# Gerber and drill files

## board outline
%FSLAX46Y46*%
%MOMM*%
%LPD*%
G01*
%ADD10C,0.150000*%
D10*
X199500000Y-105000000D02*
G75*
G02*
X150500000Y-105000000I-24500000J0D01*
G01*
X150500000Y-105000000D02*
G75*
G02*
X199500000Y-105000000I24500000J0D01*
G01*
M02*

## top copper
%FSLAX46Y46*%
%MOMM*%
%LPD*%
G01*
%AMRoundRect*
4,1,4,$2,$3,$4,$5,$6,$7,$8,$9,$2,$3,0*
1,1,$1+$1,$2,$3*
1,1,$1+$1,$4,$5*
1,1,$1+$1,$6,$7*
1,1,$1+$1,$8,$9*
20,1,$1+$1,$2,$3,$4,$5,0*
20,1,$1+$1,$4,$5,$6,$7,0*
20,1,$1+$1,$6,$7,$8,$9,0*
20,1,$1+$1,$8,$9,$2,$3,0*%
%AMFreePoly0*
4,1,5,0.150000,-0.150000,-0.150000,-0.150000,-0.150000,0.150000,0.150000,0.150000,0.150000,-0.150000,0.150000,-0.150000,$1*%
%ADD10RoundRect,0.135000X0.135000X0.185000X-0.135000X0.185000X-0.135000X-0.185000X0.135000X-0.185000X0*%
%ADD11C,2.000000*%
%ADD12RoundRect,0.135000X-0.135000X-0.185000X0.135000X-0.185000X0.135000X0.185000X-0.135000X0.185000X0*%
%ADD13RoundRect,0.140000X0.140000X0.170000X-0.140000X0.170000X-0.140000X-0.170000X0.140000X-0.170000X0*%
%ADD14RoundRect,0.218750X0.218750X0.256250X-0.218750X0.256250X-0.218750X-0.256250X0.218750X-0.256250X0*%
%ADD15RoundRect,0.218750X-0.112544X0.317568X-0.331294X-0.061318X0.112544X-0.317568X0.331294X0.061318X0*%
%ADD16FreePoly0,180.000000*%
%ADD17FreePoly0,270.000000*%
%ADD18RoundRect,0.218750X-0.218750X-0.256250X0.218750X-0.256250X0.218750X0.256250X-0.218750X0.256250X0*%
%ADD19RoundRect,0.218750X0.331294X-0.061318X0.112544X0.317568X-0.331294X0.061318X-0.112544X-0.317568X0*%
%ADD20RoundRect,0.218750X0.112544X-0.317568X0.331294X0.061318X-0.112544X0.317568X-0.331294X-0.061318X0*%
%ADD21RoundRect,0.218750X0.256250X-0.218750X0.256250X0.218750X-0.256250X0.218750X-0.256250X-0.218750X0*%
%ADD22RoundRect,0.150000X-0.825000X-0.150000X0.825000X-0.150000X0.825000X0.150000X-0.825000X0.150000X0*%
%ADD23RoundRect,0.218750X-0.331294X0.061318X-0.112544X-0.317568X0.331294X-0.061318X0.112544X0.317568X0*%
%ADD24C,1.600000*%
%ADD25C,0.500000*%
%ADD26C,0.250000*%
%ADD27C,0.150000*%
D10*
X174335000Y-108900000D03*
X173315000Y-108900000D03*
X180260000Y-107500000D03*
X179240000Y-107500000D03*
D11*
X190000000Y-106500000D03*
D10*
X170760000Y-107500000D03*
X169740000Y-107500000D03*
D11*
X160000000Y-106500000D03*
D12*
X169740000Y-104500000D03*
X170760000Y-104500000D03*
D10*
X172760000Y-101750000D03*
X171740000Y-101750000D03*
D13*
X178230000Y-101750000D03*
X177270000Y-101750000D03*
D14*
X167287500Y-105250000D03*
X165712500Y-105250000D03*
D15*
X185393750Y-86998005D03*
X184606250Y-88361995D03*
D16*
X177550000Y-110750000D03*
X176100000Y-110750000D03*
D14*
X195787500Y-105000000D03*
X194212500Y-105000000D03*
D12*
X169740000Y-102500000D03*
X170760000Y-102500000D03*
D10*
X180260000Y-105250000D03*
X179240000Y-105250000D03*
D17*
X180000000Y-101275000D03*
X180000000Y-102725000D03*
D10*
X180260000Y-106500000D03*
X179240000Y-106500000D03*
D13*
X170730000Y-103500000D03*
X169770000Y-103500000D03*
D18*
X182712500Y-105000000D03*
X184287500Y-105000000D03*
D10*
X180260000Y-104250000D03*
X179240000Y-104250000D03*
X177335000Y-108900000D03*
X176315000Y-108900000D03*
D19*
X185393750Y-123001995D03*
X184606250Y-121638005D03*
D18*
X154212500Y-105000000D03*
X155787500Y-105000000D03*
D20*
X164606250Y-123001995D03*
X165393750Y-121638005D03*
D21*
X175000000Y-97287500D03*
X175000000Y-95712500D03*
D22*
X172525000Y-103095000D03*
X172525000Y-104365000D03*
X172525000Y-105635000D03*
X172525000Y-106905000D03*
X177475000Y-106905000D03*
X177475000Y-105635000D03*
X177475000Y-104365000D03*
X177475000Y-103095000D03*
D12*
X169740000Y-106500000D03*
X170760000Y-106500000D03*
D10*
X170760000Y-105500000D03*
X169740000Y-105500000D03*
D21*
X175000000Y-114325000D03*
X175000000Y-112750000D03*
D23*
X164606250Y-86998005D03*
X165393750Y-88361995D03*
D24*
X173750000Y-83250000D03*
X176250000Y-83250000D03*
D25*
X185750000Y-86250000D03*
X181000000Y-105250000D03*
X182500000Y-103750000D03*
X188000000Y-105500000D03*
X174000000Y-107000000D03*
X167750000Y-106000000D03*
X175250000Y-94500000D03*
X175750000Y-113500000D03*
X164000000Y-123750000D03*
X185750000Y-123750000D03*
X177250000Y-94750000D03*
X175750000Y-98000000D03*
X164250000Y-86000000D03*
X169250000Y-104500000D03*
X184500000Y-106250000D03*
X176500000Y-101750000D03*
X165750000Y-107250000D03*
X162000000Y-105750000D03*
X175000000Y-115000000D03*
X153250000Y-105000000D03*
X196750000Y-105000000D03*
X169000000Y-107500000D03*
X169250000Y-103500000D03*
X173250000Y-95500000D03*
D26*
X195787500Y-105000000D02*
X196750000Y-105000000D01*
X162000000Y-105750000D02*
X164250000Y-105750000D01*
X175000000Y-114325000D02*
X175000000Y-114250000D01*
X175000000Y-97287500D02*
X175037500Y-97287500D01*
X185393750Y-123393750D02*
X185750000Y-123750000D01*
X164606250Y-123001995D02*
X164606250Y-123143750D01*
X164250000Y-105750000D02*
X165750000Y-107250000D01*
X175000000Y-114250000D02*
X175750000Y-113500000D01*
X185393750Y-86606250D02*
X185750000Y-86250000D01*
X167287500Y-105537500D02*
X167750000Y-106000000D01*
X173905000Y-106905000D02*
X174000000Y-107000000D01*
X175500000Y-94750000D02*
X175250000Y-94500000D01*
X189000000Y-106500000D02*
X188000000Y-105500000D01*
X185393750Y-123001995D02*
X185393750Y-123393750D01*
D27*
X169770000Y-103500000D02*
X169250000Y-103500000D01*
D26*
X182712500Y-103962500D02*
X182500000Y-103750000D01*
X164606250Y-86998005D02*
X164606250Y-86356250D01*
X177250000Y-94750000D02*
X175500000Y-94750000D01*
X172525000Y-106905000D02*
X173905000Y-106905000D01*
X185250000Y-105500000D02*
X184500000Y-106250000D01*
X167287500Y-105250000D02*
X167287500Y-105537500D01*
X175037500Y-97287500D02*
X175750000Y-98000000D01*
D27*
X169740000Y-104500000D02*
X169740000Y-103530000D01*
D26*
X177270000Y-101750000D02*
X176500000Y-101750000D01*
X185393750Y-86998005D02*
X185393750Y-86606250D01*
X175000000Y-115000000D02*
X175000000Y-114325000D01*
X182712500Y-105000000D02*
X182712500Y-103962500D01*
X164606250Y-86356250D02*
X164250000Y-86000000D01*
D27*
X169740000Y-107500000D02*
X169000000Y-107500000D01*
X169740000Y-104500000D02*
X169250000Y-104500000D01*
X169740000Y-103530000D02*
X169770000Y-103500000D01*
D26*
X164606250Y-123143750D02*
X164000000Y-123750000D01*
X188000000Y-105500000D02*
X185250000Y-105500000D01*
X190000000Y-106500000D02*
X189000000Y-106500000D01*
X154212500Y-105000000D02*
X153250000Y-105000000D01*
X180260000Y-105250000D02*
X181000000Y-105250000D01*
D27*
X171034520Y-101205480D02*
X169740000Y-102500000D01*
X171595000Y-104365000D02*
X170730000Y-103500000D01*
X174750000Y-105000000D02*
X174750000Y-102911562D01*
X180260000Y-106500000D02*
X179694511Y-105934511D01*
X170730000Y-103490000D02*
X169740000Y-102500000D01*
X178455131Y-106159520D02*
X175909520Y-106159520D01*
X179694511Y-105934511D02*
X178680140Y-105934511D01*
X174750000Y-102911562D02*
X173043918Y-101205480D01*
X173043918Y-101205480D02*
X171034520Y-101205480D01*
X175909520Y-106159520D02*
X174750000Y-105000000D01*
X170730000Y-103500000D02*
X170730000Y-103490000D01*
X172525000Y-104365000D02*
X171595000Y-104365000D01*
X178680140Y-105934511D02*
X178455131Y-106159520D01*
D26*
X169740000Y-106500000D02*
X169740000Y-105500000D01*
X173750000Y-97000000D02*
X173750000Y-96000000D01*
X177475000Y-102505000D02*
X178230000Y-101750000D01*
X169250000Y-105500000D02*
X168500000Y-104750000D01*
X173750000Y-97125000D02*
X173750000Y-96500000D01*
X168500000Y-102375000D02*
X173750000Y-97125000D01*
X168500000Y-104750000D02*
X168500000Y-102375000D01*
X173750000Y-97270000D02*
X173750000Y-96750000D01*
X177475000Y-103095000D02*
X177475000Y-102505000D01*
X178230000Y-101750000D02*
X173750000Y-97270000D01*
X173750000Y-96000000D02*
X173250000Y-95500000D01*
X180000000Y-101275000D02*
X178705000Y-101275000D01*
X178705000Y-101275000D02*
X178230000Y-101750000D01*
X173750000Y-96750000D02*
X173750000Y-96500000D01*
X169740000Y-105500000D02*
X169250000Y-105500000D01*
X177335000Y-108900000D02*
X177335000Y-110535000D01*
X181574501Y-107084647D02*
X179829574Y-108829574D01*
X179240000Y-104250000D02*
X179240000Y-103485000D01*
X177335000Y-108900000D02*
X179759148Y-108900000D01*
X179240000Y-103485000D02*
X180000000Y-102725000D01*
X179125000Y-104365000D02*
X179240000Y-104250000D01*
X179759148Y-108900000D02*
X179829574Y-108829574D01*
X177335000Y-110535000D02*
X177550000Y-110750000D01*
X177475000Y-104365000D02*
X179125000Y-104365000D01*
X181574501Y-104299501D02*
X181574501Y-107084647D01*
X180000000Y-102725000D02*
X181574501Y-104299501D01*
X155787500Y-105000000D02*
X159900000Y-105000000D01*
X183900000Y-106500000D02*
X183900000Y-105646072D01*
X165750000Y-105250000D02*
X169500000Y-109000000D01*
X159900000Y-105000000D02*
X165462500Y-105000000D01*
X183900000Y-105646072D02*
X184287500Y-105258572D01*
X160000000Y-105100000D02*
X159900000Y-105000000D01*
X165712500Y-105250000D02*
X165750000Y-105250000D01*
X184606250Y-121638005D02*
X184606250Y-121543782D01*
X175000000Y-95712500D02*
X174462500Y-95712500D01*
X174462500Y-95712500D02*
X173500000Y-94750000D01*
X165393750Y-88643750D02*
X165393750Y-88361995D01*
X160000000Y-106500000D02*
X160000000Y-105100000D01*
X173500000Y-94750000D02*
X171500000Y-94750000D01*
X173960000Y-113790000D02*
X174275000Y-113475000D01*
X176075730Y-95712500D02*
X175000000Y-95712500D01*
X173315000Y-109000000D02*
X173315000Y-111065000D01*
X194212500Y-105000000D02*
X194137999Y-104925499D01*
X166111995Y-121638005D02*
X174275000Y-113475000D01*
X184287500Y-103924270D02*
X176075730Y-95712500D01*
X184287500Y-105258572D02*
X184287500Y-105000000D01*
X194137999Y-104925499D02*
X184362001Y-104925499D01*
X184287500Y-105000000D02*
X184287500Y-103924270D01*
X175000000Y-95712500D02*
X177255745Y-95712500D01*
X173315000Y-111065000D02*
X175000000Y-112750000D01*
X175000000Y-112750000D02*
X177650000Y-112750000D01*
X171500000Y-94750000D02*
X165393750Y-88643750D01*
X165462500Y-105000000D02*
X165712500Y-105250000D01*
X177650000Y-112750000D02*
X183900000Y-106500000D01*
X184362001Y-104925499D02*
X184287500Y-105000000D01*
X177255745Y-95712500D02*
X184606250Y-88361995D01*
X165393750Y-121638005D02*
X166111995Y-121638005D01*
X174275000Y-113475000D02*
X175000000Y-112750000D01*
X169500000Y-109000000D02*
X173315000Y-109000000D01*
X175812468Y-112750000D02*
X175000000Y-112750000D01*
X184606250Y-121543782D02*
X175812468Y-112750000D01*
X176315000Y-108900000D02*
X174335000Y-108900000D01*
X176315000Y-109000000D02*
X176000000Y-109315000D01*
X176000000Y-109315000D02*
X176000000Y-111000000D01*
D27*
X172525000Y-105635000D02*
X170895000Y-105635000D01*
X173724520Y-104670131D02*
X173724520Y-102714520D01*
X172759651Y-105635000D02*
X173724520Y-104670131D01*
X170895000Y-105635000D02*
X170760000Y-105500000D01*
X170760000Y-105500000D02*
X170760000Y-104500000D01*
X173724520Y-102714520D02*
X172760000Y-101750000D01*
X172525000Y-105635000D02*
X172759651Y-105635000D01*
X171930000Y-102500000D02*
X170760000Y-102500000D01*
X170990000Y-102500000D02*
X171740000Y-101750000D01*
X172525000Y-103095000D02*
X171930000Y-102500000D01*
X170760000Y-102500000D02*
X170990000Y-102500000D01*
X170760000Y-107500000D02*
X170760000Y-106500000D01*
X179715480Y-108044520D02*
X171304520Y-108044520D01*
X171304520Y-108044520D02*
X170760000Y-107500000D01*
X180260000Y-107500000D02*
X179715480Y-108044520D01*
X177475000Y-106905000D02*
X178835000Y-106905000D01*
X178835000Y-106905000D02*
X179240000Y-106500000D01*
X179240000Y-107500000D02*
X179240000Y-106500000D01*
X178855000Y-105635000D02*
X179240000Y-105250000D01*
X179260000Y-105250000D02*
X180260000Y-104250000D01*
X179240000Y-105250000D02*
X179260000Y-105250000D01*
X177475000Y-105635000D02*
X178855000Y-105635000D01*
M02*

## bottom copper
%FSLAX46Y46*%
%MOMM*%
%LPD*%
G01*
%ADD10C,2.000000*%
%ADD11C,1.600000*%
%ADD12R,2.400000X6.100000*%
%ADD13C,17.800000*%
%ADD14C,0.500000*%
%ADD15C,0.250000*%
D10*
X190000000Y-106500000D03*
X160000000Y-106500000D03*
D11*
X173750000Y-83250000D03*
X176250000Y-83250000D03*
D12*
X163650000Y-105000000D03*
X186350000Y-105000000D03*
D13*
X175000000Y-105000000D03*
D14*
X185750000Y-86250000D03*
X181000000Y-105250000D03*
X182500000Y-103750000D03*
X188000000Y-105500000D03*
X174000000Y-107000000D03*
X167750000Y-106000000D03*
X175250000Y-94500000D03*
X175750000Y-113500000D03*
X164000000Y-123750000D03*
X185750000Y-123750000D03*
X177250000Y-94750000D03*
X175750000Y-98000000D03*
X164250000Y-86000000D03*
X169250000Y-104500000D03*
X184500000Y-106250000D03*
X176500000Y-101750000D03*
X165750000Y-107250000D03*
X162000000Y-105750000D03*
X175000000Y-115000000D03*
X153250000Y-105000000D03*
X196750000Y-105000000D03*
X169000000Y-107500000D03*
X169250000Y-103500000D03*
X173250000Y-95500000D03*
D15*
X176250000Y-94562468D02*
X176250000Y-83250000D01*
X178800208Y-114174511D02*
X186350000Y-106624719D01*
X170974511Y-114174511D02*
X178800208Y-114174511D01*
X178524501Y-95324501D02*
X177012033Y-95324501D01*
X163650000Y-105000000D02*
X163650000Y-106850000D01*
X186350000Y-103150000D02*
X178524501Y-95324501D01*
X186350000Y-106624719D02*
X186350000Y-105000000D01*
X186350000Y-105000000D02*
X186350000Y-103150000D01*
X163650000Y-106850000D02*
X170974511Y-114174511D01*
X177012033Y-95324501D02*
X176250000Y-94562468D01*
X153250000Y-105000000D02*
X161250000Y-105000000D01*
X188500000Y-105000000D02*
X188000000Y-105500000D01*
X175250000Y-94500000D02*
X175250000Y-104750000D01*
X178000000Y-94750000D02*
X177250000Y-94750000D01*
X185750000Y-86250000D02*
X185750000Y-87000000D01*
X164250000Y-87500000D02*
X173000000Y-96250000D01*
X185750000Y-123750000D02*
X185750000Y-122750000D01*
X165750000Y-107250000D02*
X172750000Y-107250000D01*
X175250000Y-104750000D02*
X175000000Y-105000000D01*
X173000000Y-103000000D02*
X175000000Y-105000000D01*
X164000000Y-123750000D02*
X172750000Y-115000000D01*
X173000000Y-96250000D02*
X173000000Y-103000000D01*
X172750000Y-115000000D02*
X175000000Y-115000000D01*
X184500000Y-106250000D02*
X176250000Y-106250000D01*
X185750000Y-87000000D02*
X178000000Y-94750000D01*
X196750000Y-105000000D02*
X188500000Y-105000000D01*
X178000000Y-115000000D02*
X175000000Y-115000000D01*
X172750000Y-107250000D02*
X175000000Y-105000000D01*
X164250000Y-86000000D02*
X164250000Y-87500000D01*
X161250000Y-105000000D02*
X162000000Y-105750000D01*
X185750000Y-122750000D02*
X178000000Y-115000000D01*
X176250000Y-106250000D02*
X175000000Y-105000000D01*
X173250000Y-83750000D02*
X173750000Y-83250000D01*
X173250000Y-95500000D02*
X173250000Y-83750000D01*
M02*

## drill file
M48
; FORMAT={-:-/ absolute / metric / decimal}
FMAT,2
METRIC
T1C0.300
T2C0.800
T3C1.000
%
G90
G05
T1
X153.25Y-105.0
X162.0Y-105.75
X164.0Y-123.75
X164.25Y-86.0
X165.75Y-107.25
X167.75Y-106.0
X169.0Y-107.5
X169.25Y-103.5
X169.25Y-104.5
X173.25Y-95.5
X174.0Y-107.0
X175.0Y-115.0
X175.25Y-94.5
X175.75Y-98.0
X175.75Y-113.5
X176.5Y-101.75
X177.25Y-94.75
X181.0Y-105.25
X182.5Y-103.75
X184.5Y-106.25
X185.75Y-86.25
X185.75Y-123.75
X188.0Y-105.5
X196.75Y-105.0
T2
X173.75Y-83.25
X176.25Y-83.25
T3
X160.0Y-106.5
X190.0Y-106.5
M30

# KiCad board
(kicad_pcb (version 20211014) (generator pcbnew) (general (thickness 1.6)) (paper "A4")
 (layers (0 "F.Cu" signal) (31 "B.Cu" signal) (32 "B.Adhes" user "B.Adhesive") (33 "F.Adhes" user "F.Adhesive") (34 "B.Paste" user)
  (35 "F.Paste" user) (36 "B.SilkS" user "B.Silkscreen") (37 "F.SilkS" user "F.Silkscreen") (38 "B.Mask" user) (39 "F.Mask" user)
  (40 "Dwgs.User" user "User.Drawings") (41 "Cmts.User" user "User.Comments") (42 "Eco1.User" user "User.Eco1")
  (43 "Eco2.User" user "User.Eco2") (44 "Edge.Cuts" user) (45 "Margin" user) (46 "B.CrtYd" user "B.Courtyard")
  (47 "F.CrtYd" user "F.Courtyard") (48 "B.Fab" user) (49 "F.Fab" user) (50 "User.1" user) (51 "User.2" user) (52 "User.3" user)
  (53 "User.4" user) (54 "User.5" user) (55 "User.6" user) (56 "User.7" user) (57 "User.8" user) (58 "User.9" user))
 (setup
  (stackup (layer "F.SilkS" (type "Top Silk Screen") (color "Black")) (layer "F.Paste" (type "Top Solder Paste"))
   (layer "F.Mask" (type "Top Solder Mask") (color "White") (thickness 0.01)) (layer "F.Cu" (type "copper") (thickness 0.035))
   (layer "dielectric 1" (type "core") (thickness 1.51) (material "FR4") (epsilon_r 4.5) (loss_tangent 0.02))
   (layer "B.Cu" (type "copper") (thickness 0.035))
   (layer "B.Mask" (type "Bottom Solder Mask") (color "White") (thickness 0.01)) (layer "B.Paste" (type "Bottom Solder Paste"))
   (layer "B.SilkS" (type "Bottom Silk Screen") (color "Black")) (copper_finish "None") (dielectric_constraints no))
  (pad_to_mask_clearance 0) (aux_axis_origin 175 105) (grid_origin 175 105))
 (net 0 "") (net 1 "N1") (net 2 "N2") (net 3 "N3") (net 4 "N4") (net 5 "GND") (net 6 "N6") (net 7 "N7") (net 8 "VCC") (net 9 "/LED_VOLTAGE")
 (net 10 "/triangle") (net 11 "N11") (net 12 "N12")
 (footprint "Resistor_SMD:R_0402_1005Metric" (layer "F.Cu") (at 173.825 108.9 180)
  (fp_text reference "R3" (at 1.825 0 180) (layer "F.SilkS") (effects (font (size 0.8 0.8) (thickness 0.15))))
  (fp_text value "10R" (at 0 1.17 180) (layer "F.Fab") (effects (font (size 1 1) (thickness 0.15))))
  (pad "1" smd roundrect (at -0.51 0 180) (size 0.54 0.64) (layers "F.Cu" "F.Paste" "F.Mask") (roundrect_rratio 0.25) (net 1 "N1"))
  (pad "2" smd roundrect (at 0.51 0 180) (size 0.54 0.64) (layers "F.Cu" "F.Paste" "F.Mask") (roundrect_rratio 0.25) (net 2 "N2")))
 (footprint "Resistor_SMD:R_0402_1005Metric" (layer "F.Cu") (at 179.75 107.5 180)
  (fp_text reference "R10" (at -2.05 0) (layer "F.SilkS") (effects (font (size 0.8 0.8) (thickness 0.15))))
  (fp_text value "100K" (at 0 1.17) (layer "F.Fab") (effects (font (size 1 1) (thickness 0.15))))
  (pad "1" smd roundrect (at -0.51 0 180) (size 0.54 0.64) (layers "F.Cu" "F.Paste" "F.Mask") (roundrect_rratio 0.25) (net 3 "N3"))
  (pad "2" smd roundrect (at 0.51 0 180) (size 0.54 0.64) (layers "F.Cu" "F.Paste" "F.Mask") (roundrect_rratio 0.25) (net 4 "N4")))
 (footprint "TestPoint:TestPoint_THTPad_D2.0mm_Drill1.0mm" (layer "F.Cu") (at 190 106.5)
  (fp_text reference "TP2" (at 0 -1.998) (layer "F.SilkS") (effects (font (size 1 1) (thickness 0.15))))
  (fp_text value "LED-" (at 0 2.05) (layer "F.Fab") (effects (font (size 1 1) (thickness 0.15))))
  (pad "1" thru_hole circle (at 0 0) (size 2 2) (drill 1) (layers *.Cu *.Mask) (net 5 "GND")))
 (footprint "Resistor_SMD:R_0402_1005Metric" (layer "F.Cu") (at 170.25 107.5 180)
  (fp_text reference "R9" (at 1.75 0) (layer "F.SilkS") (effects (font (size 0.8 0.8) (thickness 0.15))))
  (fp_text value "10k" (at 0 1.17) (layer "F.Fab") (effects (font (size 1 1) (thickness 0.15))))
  (pad "1" smd roundrect (at -0.51 0 180) (size 0.54 0.64) (layers "F.Cu" "F.Paste" "F.Mask") (roundrect_rratio 0.25) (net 3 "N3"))
  (pad "2" smd roundrect (at 0.51 0 180) (size 0.54 0.64) (layers "F.Cu" "F.Paste" "F.Mask") (roundrect_rratio 0.25) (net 5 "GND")))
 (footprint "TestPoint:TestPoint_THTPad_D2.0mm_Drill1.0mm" (layer "F.Cu") (at 160 106.5)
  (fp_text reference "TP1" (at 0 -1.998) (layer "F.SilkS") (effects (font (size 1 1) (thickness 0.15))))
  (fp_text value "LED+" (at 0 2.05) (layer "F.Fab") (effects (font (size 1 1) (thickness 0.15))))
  (pad "1" thru_hole circle (at 0 0) (size 2 2) (drill 1) (layers *.Cu *.Mask) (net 2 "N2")))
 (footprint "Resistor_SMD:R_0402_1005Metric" (layer "F.Cu") (at 170.25 104.5)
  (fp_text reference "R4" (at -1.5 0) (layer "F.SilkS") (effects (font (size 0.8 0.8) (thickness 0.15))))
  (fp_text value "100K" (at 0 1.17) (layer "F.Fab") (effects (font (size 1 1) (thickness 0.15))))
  (pad "1" smd roundrect (at -0.51 0) (size 0.54 0.64) (layers "F.Cu" "F.Paste" "F.Mask") (roundrect_rratio 0.25) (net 5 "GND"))
  (pad "2" smd roundrect (at 0.51 0) (size 0.54 0.64) (layers "F.Cu" "F.Paste" "F.Mask") (roundrect_rratio 0.25) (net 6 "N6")))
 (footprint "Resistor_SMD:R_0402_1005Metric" (layer "F.Cu") (at 172.25 101.75 180)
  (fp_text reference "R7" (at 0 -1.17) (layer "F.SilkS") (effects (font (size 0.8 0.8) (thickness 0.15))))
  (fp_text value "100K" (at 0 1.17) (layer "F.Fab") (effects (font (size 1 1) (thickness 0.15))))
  (pad "1" smd roundrect (at -0.51 0 180) (size 0.54 0.64) (layers "F.Cu" "F.Paste" "F.Mask") (roundrect_rratio 0.25) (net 6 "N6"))
  (pad "2" smd roundrect (at 0.51 0 180) (size 0.54 0.64) (layers "F.Cu" "F.Paste" "F.Mask") (roundrect_rratio 0.25) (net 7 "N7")))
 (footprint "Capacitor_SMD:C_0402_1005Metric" (layer "F.Cu") (at 177.75 101.75 180)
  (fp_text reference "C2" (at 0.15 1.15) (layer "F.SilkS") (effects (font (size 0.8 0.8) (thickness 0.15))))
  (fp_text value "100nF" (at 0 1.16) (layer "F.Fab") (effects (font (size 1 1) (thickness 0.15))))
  (pad "1" smd roundrect (at -0.48 0 180) (size 0.56 0.62) (layers "F.Cu" "F.Paste" "F.Mask") (roundrect_rratio 0.25) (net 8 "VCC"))
  (pad "2" smd roundrect (at 0.48 0 180) (size 0.56 0.62) (layers "F.Cu" "F.Paste" "F.Mask") (roundrect_rratio 0.25) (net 5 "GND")))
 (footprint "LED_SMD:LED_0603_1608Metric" (layer "F.Cu") (at 166.5 105.25 180)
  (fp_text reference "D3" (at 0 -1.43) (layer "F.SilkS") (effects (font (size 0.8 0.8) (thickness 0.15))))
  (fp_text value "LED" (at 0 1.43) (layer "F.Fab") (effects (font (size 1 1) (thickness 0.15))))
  (pad "1" smd roundrect (at -0.7875 0 180) (size 0.875 0.95) (layers "F.Cu" "F.Paste" "F.Mask") (roundrect_rratio 0.25) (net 5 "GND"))
  (pad "2" smd roundrect (at 0.7875 0 180) (size 0.875 0.95) (layers "F.Cu" "F.Paste" "F.Mask") (roundrect_rratio 0.25) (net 2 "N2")))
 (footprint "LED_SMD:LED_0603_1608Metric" (layer "F.Cu") (at 185 87.68 -120)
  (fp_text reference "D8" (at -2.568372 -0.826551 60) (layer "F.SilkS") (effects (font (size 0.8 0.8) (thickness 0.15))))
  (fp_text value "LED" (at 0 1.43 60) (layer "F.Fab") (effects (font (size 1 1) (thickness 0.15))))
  (pad "1" smd roundrect (at -0.7875 0 240) (size 0.875 0.95) (layers "F.Cu" "F.Paste" "F.Mask") (roundrect_rratio 0.25) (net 5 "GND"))
  (pad "2" smd roundrect (at 0.7875 0 240) (size 0.875 0.95) (layers "F.Cu" "F.Paste" "F.Mask") (roundrect_rratio 0.25) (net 2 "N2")))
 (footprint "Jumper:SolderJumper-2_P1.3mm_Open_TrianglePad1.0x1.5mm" (layer "F.Cu") (at 176.825 110.75 180)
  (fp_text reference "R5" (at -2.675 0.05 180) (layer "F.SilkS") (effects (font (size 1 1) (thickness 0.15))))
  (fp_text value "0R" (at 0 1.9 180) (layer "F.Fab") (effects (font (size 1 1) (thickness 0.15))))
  (pad "1" smd custom (at -0.725 0 180) (size 0.3 0.3) (layers "F.Cu" "F.Mask") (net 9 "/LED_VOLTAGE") (zone_connect 2)
   (options (clearance outline) (anchor rect)) (primitives))
  (pad "2" smd custom (at 0.725 0 180) (size 0.3 0.3) (layers "F.Cu" "F.Mask") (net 1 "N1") (zone_connect 2)
   (options (clearance outline) (anchor rect)) (primitives)))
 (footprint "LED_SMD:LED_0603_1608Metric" (layer "F.Cu") (at 195 105 180)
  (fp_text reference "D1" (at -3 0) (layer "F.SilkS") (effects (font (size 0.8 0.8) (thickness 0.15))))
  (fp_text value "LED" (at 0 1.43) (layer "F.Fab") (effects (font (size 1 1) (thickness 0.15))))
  (pad "1" smd roundrect (at -0.7875 0 180) (size 0.875 0.95) (layers "F.Cu" "F.Paste" "F.Mask") (roundrect_rratio 0.25) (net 5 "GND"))
  (pad "2" smd roundrect (at 0.7875 0 180) (size 0.875 0.95) (layers "F.Cu" "F.Paste" "F.Mask") (roundrect_rratio 0.25) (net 2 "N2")))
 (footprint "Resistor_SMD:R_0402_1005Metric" (layer "F.Cu") (at 170.25 102.5)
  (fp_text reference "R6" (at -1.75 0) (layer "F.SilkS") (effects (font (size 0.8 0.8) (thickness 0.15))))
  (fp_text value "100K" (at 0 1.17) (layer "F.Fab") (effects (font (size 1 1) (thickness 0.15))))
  (pad "1" smd roundrect (at -0.51 0) (size 0.54 0.64) (layers "F.Cu" "F.Paste" "F.Mask") (roundrect_rratio 0.25) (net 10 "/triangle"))
  (pad "2" smd roundrect (at 0.51 0) (size 0.54 0.64) (layers "F.Cu" "F.Paste" "F.Mask") (roundrect_rratio 0.25) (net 7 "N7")))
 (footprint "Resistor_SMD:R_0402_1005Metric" (layer "F.Cu") (at 179.75 105.25 180)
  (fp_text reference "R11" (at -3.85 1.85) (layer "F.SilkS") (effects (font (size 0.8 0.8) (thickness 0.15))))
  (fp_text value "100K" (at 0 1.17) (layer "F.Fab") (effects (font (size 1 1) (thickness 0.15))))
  (pad "1" smd roundrect (at -0.51 0 180) (size 0.54 0.64) (layers "F.Cu" "F.Paste" "F.Mask") (roundrect_rratio 0.25) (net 5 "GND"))
  (pad "2" smd roundrect (at 0.51 0 180) (size 0.54 0.64) (layers "F.Cu" "F.Paste" "F.Mask") (roundrect_rratio 0.25) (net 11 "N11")))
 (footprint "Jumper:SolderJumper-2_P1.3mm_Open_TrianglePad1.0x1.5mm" (layer "F.Cu") (at 180 102 -90)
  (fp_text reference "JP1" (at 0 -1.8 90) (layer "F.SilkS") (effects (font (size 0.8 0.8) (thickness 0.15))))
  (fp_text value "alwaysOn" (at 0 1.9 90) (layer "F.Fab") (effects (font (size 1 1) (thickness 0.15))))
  (pad "1" smd custom (at -0.725 0 270) (size 0.3 0.3) (layers "F.Cu" "F.Mask") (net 8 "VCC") (zone_connect 2)
   (options (clearance outline) (anchor rect)) (primitives))
  (pad "2" smd custom (at 0.725 0 270) (size 0.3 0.3) (layers "F.Cu" "F.Mask") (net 9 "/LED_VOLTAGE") (zone_connect 2)
   (options (clearance outline) (anchor rect)) (primitives)))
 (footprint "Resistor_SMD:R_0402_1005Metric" (layer "F.Cu") (at 179.75 106.5 180)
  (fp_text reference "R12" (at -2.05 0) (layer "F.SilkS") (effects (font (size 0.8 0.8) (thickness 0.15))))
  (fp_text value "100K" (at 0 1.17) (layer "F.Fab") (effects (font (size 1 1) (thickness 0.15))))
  (pad "1" smd roundrect (at -0.51 0 180) (size 0.54 0.64) (layers "F.Cu" "F.Paste" "F.Mask") (roundrect_rratio 0.25) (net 10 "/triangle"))
  (pad "2" smd roundrect (at 0.51 0 180) (size 0.54 0.64) (layers "F.Cu" "F.Paste" "F.Mask") (roundrect_rratio 0.25) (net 4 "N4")))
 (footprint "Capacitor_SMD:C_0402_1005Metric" (layer "F.Cu") (at 170.25 103.5 180)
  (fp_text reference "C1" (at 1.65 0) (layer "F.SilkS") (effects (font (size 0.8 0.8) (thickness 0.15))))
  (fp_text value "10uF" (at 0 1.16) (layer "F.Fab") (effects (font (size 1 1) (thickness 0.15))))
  (pad "1" smd roundrect (at -0.48 0 180) (size 0.56 0.62) (layers "F.Cu" "F.Paste" "F.Mask") (roundrect_rratio 0.25) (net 10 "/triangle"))
  (pad "2" smd roundrect (at 0.48 0 180) (size 0.56 0.62) (layers "F.Cu" "F.Paste" "F.Mask") (roundrect_rratio 0.25) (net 5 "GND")))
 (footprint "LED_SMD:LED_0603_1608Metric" (layer "F.Cu") (at 183.5 105)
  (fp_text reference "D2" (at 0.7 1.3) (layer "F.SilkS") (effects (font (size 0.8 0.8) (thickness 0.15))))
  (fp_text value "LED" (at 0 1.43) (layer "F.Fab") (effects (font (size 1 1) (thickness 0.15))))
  (pad "1" smd roundrect (at -0.7875 0) (size 0.875 0.95) (layers "F.Cu" "F.Paste" "F.Mask") (roundrect_rratio 0.25) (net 5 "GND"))
  (pad "2" smd roundrect (at 0.7875 0) (size 0.875 0.95) (layers "F.Cu" "F.Paste" "F.Mask") (roundrect_rratio 0.25) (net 2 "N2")))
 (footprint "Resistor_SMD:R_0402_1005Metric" (layer "F.Cu") (at 179.75 104.25 180)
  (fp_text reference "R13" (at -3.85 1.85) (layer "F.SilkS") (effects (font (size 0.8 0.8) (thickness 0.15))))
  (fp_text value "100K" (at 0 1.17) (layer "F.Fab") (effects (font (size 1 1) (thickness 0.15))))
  (pad "1" smd roundrect (at -0.51 0 180) (size 0.54 0.64) (layers "F.Cu" "F.Paste" "F.Mask") (roundrect_rratio 0.25) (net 11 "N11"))
  (pad "2" smd roundrect (at 0.51 0 180) (size 0.54 0.64) (layers "F.Cu" "F.Paste" "F.Mask") (roundrect_rratio 0.25) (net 9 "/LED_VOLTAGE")))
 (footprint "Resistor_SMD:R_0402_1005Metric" (layer "F.Cu") (at 176.825 108.9 180)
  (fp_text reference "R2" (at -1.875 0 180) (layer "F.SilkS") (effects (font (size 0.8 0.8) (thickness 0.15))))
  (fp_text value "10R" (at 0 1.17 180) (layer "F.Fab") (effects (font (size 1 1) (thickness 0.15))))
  (pad "1" smd roundrect (at -0.51 0 180) (size 0.54 0.64) (layers "F.Cu" "F.Paste" "F.Mask") (roundrect_rratio 0.25) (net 9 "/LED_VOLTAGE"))
  (pad "2" smd roundrect (at 0.51 0 180) (size 0.54 0.64) (layers "F.Cu" "F.Paste" "F.Mask") (roundrect_rratio 0.25) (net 1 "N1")))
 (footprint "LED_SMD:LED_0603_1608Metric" (layer "F.Cu") (at 185 122.32 120)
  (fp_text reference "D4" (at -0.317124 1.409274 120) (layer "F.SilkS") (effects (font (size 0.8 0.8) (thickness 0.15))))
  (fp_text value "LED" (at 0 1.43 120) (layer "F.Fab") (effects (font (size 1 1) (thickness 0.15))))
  (pad "1" smd roundrect (at -0.7875 0 120) (size 0.875 0.95) (layers "F.Cu" "F.Paste" "F.Mask") (roundrect_rratio 0.25) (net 5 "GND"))
  (pad "2" smd roundrect (at 0.7875 0 120) (size 0.875 0.95) (layers "F.Cu" "F.Paste" "F.Mask") (roundrect_rratio 0.25) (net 2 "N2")))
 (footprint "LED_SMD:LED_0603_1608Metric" (layer "F.Cu") (at 155 105)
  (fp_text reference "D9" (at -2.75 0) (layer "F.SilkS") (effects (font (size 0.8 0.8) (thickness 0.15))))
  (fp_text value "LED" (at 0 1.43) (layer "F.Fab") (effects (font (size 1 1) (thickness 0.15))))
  (pad "1" smd roundrect (at -0.7875 0) (size 0.875 0.95) (layers "F.Cu" "F.Paste" "F.Mask") (roundrect_rratio 0.25) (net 5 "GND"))
  (pad "2" smd roundrect (at 0.7875 0) (size 0.875 0.95) (layers "F.Cu" "F.Paste" "F.Mask") (roundrect_rratio 0.25) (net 2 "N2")))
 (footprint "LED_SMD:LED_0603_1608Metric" (layer "F.Cu") (at 165 122.32 60)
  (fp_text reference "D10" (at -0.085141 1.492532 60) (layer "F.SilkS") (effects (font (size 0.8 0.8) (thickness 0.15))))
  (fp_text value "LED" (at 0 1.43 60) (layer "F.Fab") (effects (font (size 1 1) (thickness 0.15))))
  (pad "1" smd roundrect (at -0.7875 0 60) (size 0.875 0.95) (layers "F.Cu" "F.Paste" "F.Mask") (roundrect_rratio 0.25) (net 5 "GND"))
  (pad "2" smd roundrect (at 0.7875 0 60) (size 0.875 0.95) (layers "F.Cu" "F.Paste" "F.Mask") (roundrect_rratio 0.25) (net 2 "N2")))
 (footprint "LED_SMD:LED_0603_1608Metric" (layer "F.Cu") (at 175 96.5 90)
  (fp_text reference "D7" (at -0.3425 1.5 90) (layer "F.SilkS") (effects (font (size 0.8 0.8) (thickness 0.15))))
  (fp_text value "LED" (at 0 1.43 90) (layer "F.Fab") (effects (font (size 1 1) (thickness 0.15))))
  (pad "1" smd roundrect (at -0.7875 0 90) (size 0.875 0.95) (layers "F.Cu" "F.Paste" "F.Mask") (roundrect_rratio 0.25) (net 5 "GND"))
  (pad "2" smd roundrect (at 0.7875 0 90) (size 0.875 0.95) (layers "F.Cu" "F.Paste" "F.Mask") (roundrect_rratio 0.25) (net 2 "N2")))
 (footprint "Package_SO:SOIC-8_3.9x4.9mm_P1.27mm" (layer "F.Cu") (at 175 105)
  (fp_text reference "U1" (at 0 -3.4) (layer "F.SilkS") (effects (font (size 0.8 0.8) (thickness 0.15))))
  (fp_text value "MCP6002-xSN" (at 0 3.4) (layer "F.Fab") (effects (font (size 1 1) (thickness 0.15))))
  (pad "1" smd roundrect (at -2.475 -1.905) (size 1.95 0.6) (layers "F.Cu" "F.Paste" "F.Mask") (roundrect_rratio 0.25) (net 7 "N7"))
  (pad "2" smd roundrect (at -2.475 -0.635) (size 1.95 0.6) (layers "F.Cu" "F.Paste" "F.Mask") (roundrect_rratio 0.25) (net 10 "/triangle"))
  (pad "3" smd roundrect (at -2.475 0.635) (size 1.95 0.6) (layers "F.Cu" "F.Paste" "F.Mask") (roundrect_rratio 0.25) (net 6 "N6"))
  (pad "4" smd roundrect (at -2.475 1.905) (size 1.95 0.6) (layers "F.Cu" "F.Paste" "F.Mask") (roundrect_rratio 0.25) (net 5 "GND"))
  (pad "5" smd roundrect (at 2.475 1.905) (size 1.95 0.6) (layers "F.Cu" "F.Paste" "F.Mask") (roundrect_rratio 0.25) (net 4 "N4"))
  (pad "6" smd roundrect (at 2.475 0.635) (size 1.95 0.6) (layers "F.Cu" "F.Paste" "F.Mask") (roundrect_rratio 0.25) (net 11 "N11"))
  (pad "7" smd roundrect (at 2.475 -0.635) (size 1.95 0.6) (layers "F.Cu" "F.Paste" "F.Mask") (roundrect_rratio 0.25) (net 9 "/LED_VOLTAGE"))
  (pad "8" smd roundrect (at 2.475 -1.905) (size 1.95 0.6) (layers "F.Cu" "F.Paste" "F.Mask") (roundrect_rratio 0.25) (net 8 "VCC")))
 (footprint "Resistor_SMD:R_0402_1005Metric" (layer "F.Cu") (at 170.25 106.5)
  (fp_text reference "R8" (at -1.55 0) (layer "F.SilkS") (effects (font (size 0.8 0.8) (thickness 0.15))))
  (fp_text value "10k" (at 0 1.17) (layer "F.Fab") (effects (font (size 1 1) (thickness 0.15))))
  (pad "1" smd roundrect (at -0.51 0) (size 0.54 0.64) (layers "F.Cu" "F.Paste" "F.Mask") (roundrect_rratio 0.25) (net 8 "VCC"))
  (pad "2" smd roundrect (at 0.51 0) (size 0.54 0.64) (layers "F.Cu" "F.Paste" "F.Mask") (roundrect_rratio 0.25) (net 3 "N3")))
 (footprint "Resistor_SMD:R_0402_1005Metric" (layer "F.Cu") (at 170.25 105.5 180)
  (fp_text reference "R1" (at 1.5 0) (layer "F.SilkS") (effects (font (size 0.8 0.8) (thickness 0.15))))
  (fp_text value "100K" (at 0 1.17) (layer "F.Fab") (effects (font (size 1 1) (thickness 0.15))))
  (pad "1" smd roundrect (at -0.51 0 180) (size 0.54 0.64) (layers "F.Cu" "F.Paste" "F.Mask") (roundrect_rratio 0.25) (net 6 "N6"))
  (pad "2" smd roundrect (at 0.51 0 180) (size 0.54 0.64) (layers "F.Cu" "F.Paste" "F.Mask") (roundrect_rratio 0.25) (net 8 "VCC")))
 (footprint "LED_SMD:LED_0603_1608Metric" (layer "F.Cu") (at 175 113.5375 90)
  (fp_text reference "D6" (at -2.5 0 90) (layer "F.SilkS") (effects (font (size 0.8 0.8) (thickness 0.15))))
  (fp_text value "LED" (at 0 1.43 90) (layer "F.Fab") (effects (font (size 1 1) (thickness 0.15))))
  (pad "1" smd roundrect (at -0.7875 0 90) (size 0.875 0.95) (layers "F.Cu" "F.Paste" "F.Mask") (roundrect_rratio 0.25) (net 5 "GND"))
  (pad "2" smd roundrect (at 0.7875 0 90) (size 0.875 0.95) (layers "F.Cu" "F.Paste" "F.Mask") (roundrect_rratio 0.25) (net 2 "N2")))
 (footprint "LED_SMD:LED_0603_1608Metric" (layer "F.Cu") (at 165 87.68 -60)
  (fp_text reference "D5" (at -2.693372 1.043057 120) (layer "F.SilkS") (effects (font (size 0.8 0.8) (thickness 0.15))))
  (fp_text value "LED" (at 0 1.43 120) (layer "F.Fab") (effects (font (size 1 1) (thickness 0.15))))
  (pad "1" smd roundrect (at -0.7875 0 300) (size 0.875 0.95) (layers "F.Cu" "F.Paste" "F.Mask") (roundrect_rratio 0.25) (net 5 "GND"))
  (pad "2" smd roundrect (at 0.7875 0 300) (size 0.875 0.95) (layers "F.Cu" "F.Paste" "F.Mask") (roundrect_rratio 0.25) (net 2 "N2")))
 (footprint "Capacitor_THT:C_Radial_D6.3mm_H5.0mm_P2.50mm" (layer "B.Cu") (at 173.75 83.25)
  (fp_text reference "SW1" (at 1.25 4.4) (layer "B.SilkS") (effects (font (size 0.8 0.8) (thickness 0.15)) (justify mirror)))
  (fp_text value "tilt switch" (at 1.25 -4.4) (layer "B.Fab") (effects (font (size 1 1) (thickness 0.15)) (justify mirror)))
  (pad "1" thru_hole circle (at 0 0) (size 1.6 1.6) (drill 0.8) (layers *.Cu *.Mask) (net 8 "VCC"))
  (pad "2" thru_hole circle (at 2.5 0) (size 1.6 1.6) (drill 0.8) (layers *.Cu *.Mask) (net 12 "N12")))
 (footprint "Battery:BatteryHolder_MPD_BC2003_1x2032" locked (layer "B.Cu") (at 175 105 180)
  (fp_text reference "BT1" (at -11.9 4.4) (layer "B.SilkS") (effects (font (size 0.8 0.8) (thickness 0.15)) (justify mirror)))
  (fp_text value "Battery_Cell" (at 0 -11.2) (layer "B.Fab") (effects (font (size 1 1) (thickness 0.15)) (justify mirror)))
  (pad "1" smd rect locked (at 11.35 0 180) (size 2.4 6.1) (layers "B.Cu" "B.Paste" "B.Mask") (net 12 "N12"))
  (pad "1" smd rect locked (at -11.35 0 180) (size 2.4 6.1) (layers "B.Cu" "B.Paste" "B.Mask") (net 12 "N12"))
  (pad "2" smd circle locked (at 0 0 180) (size 17.8 17.8) (layers "B.Cu" "B.Mask") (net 5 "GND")))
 (gr_circle (center 175 105) (end 199.5 105) (layer "Edge.Cuts") (width 0.15) (fill none))
 (segment (start 176.25 94.562468) (end 176.25 83.25) (width 0.25) (layer "B.Cu") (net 12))
 (segment (start 178.800208 114.174511) (end 186.35 106.624719) (width 0.25) (layer "B.Cu") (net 12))
 (segment (start 170.974511 114.174511) (end 178.800208 114.174511) (width 0.25) (layer "B.Cu") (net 12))
 (segment (start 178.524501 95.324501) (end 177.012033 95.324501) (width 0.25) (layer "B.Cu") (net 12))
 (segment (start 163.65 105) (end 163.65 106.85) (width 0.25) (layer "B.Cu") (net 12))
 (segment (start 186.35 103.15) (end 178.524501 95.324501) (width 0.25) (layer "B.Cu") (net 12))
 (segment (start 186.35 106.624719) (end 186.35 105) (width 0.25) (layer "B.Cu") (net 12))
 (segment (start 186.35 105) (end 186.35 103.15) (width 0.25) (layer "B.Cu") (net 12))
 (segment (start 163.65 106.85) (end 170.974511 114.174511) (width 0.25) (layer "B.Cu") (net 12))
 (segment (start 177.012033 95.324501) (end 176.25 94.562468) (width 0.25) (layer "B.Cu") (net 12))
 (segment (start 195.7875 105) (end 196.75 105) (width 0.25) (layer "F.Cu") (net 5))
 (segment (start 162 105.75) (end 164.25 105.75) (width 0.25) (layer "F.Cu") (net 5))
 (segment (start 175 114.325) (end 175 114.25) (width 0.25) (layer "F.Cu") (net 5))
 (segment (start 175 97.2875) (end 175.0375 97.2875) (width 0.25) (layer "F.Cu") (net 5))
 (segment (start 185.39375 123.39375) (end 185.75 123.75) (width 0.25) (layer "F.Cu") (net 5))
 (segment (start 164.60625 123.001995) (end 164.60625 123.14375) (width 0.25) (layer "F.Cu") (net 5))
 (segment (start 164.25 105.75) (end 165.75 107.25) (width 0.25) (layer "F.Cu") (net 5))
 (segment (start 175 114.25) (end 175.75 113.5) (width 0.25) (layer "F.Cu") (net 5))
 (segment (start 185.39375 86.60625) (end 185.75 86.25) (width 0.25) (layer "F.Cu") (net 5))
 (segment (start 167.2875 105.5375) (end 167.75 106) (width 0.25) (layer "F.Cu") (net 5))
 (segment (start 173.905 106.905) (end 174 107) (width 0.25) (layer "F.Cu") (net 5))
 (segment (start 175.5 94.75) (end 175.25 94.5) (width 0.25) (layer "F.Cu") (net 5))
 (segment (start 189 106.5) (end 188 105.5) (width 0.25) (layer "F.Cu") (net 5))
 (segment (start 185.39375 123.001995) (end 185.39375 123.39375) (width 0.25) (layer "F.Cu") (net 5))
 (segment (start 169.77 103.5) (end 169.25 103.5) (width 0.15) (layer "F.Cu") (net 5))
 (segment (start 182.7125 103.9625) (end 182.5 103.75) (width 0.25) (layer "F.Cu") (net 5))
 (segment (start 164.60625 86.998005) (end 164.60625 86.35625) (width 0.25) (layer "F.Cu") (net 5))
 (segment (start 177.25 94.75) (end 175.5 94.75) (width 0.25) (layer "F.Cu") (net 5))
 (segment (start 172.525 106.905) (end 173.905 106.905) (width 0.25) (layer "F.Cu") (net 5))
 (segment (start 185.25 105.5) (end 184.5 106.25) (width 0.25) (layer "F.Cu") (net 5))
 (segment (start 167.2875 105.25) (end 167.2875 105.5375) (width 0.25) (layer "F.Cu") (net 5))
 (segment (start 175.0375 97.2875) (end 175.75 98) (width 0.25) (layer "F.Cu") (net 5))
 (segment (start 169.74 104.5) (end 169.74 103.53) (width 0.15) (layer "F.Cu") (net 5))
 (segment (start 177.27 101.75) (end 176.5 101.75) (width 0.25) (layer "F.Cu") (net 5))
 (segment (start 185.39375 86.998005) (end 185.39375 86.60625) (width 0.25) (layer "F.Cu") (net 5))
 (segment (start 175 115) (end 175 114.325) (width 0.25) (layer "F.Cu") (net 5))
 (segment (start 182.7125 105) (end 182.7125 103.9625) (width 0.25) (layer "F.Cu") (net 5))
 (segment (start 164.60625 86.35625) (end 164.25 86) (width 0.25) (layer "F.Cu") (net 5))
 (segment (start 169.74 107.5) (end 169 107.5) (width 0.15) (layer "F.Cu") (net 5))
 (segment (start 169.74 104.5) (end 169.25 104.5) (width 0.15) (layer "F.Cu") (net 5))
 (segment (start 169.74 103.53) (end 169.77 103.5) (width 0.15) (layer "F.Cu") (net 5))
 (segment (start 164.60625 123.14375) (end 164 123.75) (width 0.25) (layer "F.Cu") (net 5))
 (segment (start 188 105.5) (end 185.25 105.5) (width 0.25) (layer "F.Cu") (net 5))
 (segment (start 190 106.5) (end 189 106.5) (width 0.25) (layer "F.Cu") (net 5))
 (segment (start 154.2125 105) (end 153.25 105) (width 0.25) (layer "F.Cu") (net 5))
 (segment (start 180.26 105.25) (end 181 105.25) (width 0.25) (layer "F.Cu") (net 5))
 (via (at 185.75 86.25) (size 0.5) (drill 0.3) (layers "F.Cu" "B.Cu") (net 5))
 (via (at 181 105.25) (size 0.5) (drill 0.3) (layers "F.Cu" "B.Cu") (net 5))
 (via (at 182.5 103.75) (size 0.5) (drill 0.3) (layers "F.Cu" "B.Cu") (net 5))
 (via (at 188 105.5) (size 0.5) (drill 0.3) (layers "F.Cu" "B.Cu") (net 5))
 (via (at 174 107) (size 0.5) (drill 0.3) (layers "F.Cu" "B.Cu") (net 5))
 (via (at 167.75 106) (size 0.5) (drill 0.3) (layers "F.Cu" "B.Cu") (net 5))
 (via (at 175.25 94.5) (size 0.5) (drill 0.3) (layers "F.Cu" "B.Cu") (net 5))
 (via (at 175.75 113.5) (size 0.5) (drill 0.3) (layers "F.Cu" "B.Cu") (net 5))
 (via (at 164 123.75) (size 0.5) (drill 0.3) (layers "F.Cu" "B.Cu") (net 5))
 (via (at 185.75 123.75) (size 0.5) (drill 0.3) (layers "F.Cu" "B.Cu") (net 5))
 (via (at 177.25 94.75) (size 0.5) (drill 0.3) (layers "F.Cu" "B.Cu") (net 5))
 (via (at 175.75 98) (size 0.5) (drill 0.3) (layers "F.Cu" "B.Cu") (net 5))
 (via (at 164.25 86) (size 0.5) (drill 0.3) (layers "F.Cu" "B.Cu") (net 5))
 (via (at 169.25 104.5) (size 0.5) (drill 0.3) (layers "F.Cu" "B.Cu") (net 5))
 (via (at 184.5 106.25) (size 0.5) (drill 0.3) (layers "F.Cu" "B.Cu") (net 5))
 (via (at 176.5 101.75) (size 0.5) (drill 0.3) (layers "F.Cu" "B.Cu") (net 5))
 (via (at 165.75 107.25) (size 0.5) (drill 0.3) (layers "F.Cu" "B.Cu") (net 5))
 (via (at 162 105.75) (size 0.5) (drill 0.3) (layers "F.Cu" "B.Cu") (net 5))
 (via (at 175 115) (size 0.5) (drill 0.3) (layers "F.Cu" "B.Cu") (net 5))
 (via (at 153.25 105) (size 0.5) (drill 0.3) (layers "F.Cu" "B.Cu") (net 5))
 (via (at 196.75 105) (size 0.5) (drill 0.3) (layers "F.Cu" "B.Cu") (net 5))
 (via (at 169 107.5) (size 0.5) (drill 0.3) (layers "F.Cu" "B.Cu") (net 5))
 (via (at 169.25 103.5) (size 0.5) (drill 0.3) (layers "F.Cu" "B.Cu") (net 5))
 (segment (start 153.25 105) (end 161.25 105) (width 0.25) (layer "B.Cu") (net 5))
 (segment (start 188.5 105) (end 188 105.5) (width 0.25) (layer "B.Cu") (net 5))
 (segment (start 175.25 94.5) (end 175.25 104.75) (width 0.25) (layer "B.Cu") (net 5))
 (segment (start 178 94.75) (end 177.25 94.75) (width 0.25) (layer "B.Cu") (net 5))
 (segment (start 185.75 86.25) (end 185.75 87) (width 0.25) (layer "B.Cu") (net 5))
 (segment (start 164.25 87.5) (end 173 96.25) (width 0.25) (layer "B.Cu") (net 5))
 (segment (start 185.75 123.75) (end 185.75 122.75) (width 0.25) (layer "B.Cu") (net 5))
 (segment (start 165.75 107.25) (end 172.75 107.25) (width 0.25) (layer "B.Cu") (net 5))
 (segment (start 175.25 104.75) (end 175 105) (width 0.25) (layer "B.Cu") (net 5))
 (segment (start 173 103) (end 175 105) (width 0.25) (layer "B.Cu") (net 5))
 (segment (start 164 123.75) (end 172.75 115) (width 0.25) (layer "B.Cu") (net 5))
 (segment (start 173 96.25) (end 173 103) (width 0.25) (layer "B.Cu") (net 5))
 (segment (start 172.75 115) (end 175 115) (width 0.25) (layer "B.Cu") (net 5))
 (segment (start 184.5 106.25) (end 176.25 106.25) (width 0.25) (layer "B.Cu") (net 5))
 (segment (start 185.75 87) (end 178 94.75) (width 0.25) (layer "B.Cu") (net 5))
 (segment (start 196.75 105) (end 188.5 105) (width 0.25) (layer "B.Cu") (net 5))
 (segment (start 178 115) (end 175 115) (width 0.25) (layer "B.Cu") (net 5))
 (segment (start 172.75 107.25) (end 175 105) (width 0.25) (layer "B.Cu") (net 5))
 (segment (start 164.25 86) (end 164.25 87.5) (width 0.25) (layer "B.Cu") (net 5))
 (segment (start 161.25 105) (end 162 105.75) (width 0.25) (layer "B.Cu") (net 5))
 (segment (start 185.75 122.75) (end 178 115) (width 0.25) (layer "B.Cu") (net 5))
 (segment (start 176.25 106.25) (end 175 105) (width 0.25) (layer "B.Cu") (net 5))
 (segment (start 171.03452 101.20548) (end 169.74 102.5) (width 0.15) (layer "F.Cu") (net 10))
 (segment (start 171.595 104.365) (end 170.73 103.5) (width 0.15) (layer "F.Cu") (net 10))
 (segment (start 174.75 105) (end 174.75 102.911562) (width 0.15) (layer "F.Cu") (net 10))
 (segment (start 180.26 106.5) (end 179.694511 105.934511) (width 0.15) (layer "F.Cu") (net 10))
 (segment (start 170.73 103.49) (end 169.74 102.5) (width 0.15) (layer "F.Cu") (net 10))
 (segment (start 178.455131 106.15952) (end 175.90952 106.15952) (width 0.15) (layer "F.Cu") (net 10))
 (segment (start 179.694511 105.934511) (end 178.68014 105.934511) (width 0.15) (layer "F.Cu") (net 10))
 (segment (start 174.75 102.911562) (end 173.043918 101.20548) (width 0.15) (layer "F.Cu") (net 10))
 (segment (start 173.043918 101.20548) (end 171.03452 101.20548) (width 0.15) (layer "F.Cu") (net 10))
 (segment (start 175.90952 106.15952) (end 174.75 105) (width 0.15) (layer "F.Cu") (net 10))
 (segment (start 170.73 103.5) (end 170.73 103.49) (width 0.15) (layer "F.Cu") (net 10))
 (segment (start 172.525 104.365) (end 171.595 104.365) (width 0.15) (layer "F.Cu") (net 10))
 (segment (start 178.68014 105.934511) (end 178.455131 106.15952) (width 0.15) (layer "F.Cu") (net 10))
 (segment (start 169.74 106.5) (end 169.74 105.5) (width 0.25) (layer "F.Cu") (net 8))
 (segment (start 173.75 97) (end 173.75 96) (width 0.25) (layer "F.Cu") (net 8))
 (segment (start 177.475 102.505) (end 178.23 101.75) (width 0.25) (layer "F.Cu") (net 8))
 (segment (start 169.25 105.5) (end 168.5 104.75) (width 0.25) (layer "F.Cu") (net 8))
 (segment (start 173.75 97.125) (end 173.75 96.5) (width 0.25) (layer "F.Cu") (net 8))
 (segment (start 168.5 102.375) (end 173.75 97.125) (width 0.25) (layer "F.Cu") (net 8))
 (segment (start 168.5 104.75) (end 168.5 102.375) (width 0.25) (layer "F.Cu") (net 8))
 (segment (start 173.75 97.27) (end 173.75 96.75) (width 0.25) (layer "F.Cu") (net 8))
 (segment (start 177.475 103.095) (end 177.475 102.505) (width 0.25) (layer "F.Cu") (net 8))
 (segment (start 178.23 101.75) (end 173.75 97.27) (width 0.25) (layer "F.Cu") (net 8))
 (segment (start 173.75 96) (end 173.25 95.5) (width 0.25) (layer "F.Cu") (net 8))
 (segment (start 180 101.275) (end 178.705 101.275) (width 0.25) (layer "F.Cu") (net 8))
 (segment (start 178.705 101.275) (end 178.23 101.75) (width 0.25) (layer "F.Cu") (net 8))
 (segment (start 173.75 96.75) (end 173.75 96.5) (width 0.25) (layer "F.Cu") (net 8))
 (segment (start 169.74 105.5) (end 169.25 105.5) (width 0.25) (layer "F.Cu") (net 8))
 (via (at 173.25 95.5) (size 0.5) (drill 0.3) (layers "F.Cu" "B.Cu") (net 8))
 (segment (start 173.25 83.75) (end 173.75 83.25) (width 0.25) (layer "B.Cu") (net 8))
 (segment (start 173.25 95.5) (end 173.25 83.75) (width 0.25) (layer "B.Cu") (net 8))
 (segment (start 177.335 108.9) (end 177.335 110.535) (width 0.25) (layer "F.Cu") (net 9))
 (segment (start 181.574501 107.084647) (end 179.829574 108.829574) (width 0.25) (layer "F.Cu") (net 9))
 (segment (start 179.24 104.25) (end 179.24 103.485) (width 0.25) (layer "F.Cu") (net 9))
 (segment (start 177.335 108.9) (end 179.759148 108.9) (width 0.25) (layer "F.Cu") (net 9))
 (segment (start 179.24 103.485) (end 180 102.725) (width 0.25) (layer "F.Cu") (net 9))
 (segment (start 179.125 104.365) (end 179.24 104.25) (width 0.25) (layer "F.Cu") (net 9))
 (segment (start 179.759148 108.9) (end 179.829574 108.829574) (width 0.25) (layer "F.Cu") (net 9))
 (segment (start 177.335 110.535) (end 177.55 110.75) (width 0.25) (layer "F.Cu") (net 9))
 (segment (start 177.475 104.365) (end 179.125 104.365) (width 0.25) (layer "F.Cu") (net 9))
 (segment (start 181.574501 104.299501) (end 181.574501 107.084647) (width 0.25) (layer "F.Cu") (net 9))
 (segment (start 180 102.725) (end 181.574501 104.299501) (width 0.25) (layer "F.Cu") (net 9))
 (segment (start 155.7875 105) (end 159.9 105) (width 0.25) (layer "F.Cu") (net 2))
 (segment (start 183.9 106.5) (end 183.9 105.646072) (width 0.25) (layer "F.Cu") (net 2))
 (segment (start 165.75 105.25) (end 169.5 109) (width 0.25) (layer "F.Cu") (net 2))
 (segment (start 159.9 105) (end 165.4625 105) (width 0.25) (layer "F.Cu") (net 2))
 (segment (start 183.9 105.646072) (end 184.2875 105.258572) (width 0.25) (layer "F.Cu") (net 2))
 (segment (start 160 105.1) (end 159.9 105) (width 0.25) (layer "F.Cu") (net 2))
 (segment (start 165.7125 105.25) (end 165.75 105.25) (width 0.25) (layer "F.Cu") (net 2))
 (segment (start 184.60625 121.638005) (end 184.60625 121.543782) (width 0.25) (layer "F.Cu") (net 2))
 (segment (start 175 95.7125) (end 174.4625 95.7125) (width 0.25) (layer "F.Cu") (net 2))
 (segment (start 174.4625 95.7125) (end 173.5 94.75) (width 0.25) (layer "F.Cu") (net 2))
 (segment (start 165.39375 88.64375) (end 165.39375 88.361995) (width 0.25) (layer "F.Cu") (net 2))
 (segment (start 160 106.5) (end 160 105.1) (width 0.25) (layer "F.Cu") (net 2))
 (segment (start 173.5 94.75) (end 171.5 94.75) (width 0.25) (layer "F.Cu") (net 2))
 (segment (start 173.96 113.79) (end 174.275 113.475) (width 0.25) (layer "F.Cu") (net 2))
 (segment (start 176.07573 95.7125) (end 175 95.7125) (width 0.25) (layer "F.Cu") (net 2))
 (segment (start 173.315 109) (end 173.315 111.065) (width 0.25) (layer "F.Cu") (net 2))
 (segment (start 194.2125 105) (end 194.137999 104.925499) (width 0.25) (layer "F.Cu") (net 2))
 (segment (start 166.111995 121.638005) (end 174.275 113.475) (width 0.25) (layer "F.Cu") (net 2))
 (segment (start 184.2875 103.92427) (end 176.07573 95.7125) (width 0.25) (layer "F.Cu") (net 2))
 (segment (start 184.2875 105.258572) (end 184.2875 105) (width 0.25) (layer "F.Cu") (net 2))
 (segment (start 194.137999 104.925499) (end 184.362001 104.925499) (width 0.25) (layer "F.Cu") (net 2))
 (segment (start 184.2875 105) (end 184.2875 103.92427) (width 0.25) (layer "F.Cu") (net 2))
 (segment (start 175 95.7125) (end 177.255745 95.7125) (width 0.25) (layer "F.Cu") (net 2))
 (segment (start 173.315 111.065) (end 175 112.75) (width 0.25) (layer "F.Cu") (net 2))
 (segment (start 175 112.75) (end 177.65 112.75) (width 0.25) (layer "F.Cu") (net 2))
 (segment (start 171.5 94.75) (end 165.39375 88.64375) (width 0.25) (layer "F.Cu") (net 2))
 (segment (start 165.4625 105) (end 165.7125 105.25) (width 0.25) (layer "F.Cu") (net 2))
 (segment (start 177.65 112.75) (end 183.9 106.5) (width 0.25) (layer "F.Cu") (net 2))
 (segment (start 184.362001 104.925499) (end 184.2875 105) (width 0.25) (layer "F.Cu") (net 2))
 (segment (start 177.255745 95.7125) (end 184.60625 88.361995) (width 0.25) (layer "F.Cu") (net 2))
 (segment (start 165.39375 121.638005) (end 166.111995 121.638005) (width 0.25) (layer "F.Cu") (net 2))
 (segment (start 174.275 113.475) (end 175 112.75) (width 0.25) (layer "F.Cu") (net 2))
 (segment (start 169.5 109) (end 173.315 109) (width 0.25) (layer "F.Cu") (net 2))
 (segment (start 175.812468 112.75) (end 175 112.75) (width 0.25) (layer "F.Cu") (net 2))
 (segment (start 184.60625 121.543782) (end 175.812468 112.75) (width 0.25) (layer "F.Cu") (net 2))
 (segment (start 176.315 108.9) (end 174.335 108.9) (width 0.25) (layer "F.Cu") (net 1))
 (segment (start 176.315 109) (end 176 109.315) (width 0.25) (layer "F.Cu") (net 1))
 (segment (start 176 109.315) (end 176 111) (width 0.25) (layer "F.Cu") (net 1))
 (segment (start 172.525 105.635) (end 170.895 105.635) (width 0.15) (layer "F.Cu") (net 6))
 (segment (start 173.72452 104.670131) (end 173.72452 102.71452) (width 0.15) (layer "F.Cu") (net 6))
 (segment (start 172.759651 105.635) (end 173.72452 104.670131) (width 0.15) (layer "F.Cu") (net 6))
 (segment (start 170.895 105.635) (end 170.76 105.5) (width 0.15) (layer "F.Cu") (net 6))
 (segment (start 170.76 105.5) (end 170.76 104.5) (width 0.15) (layer "F.Cu") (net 6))
 (segment (start 173.72452 102.71452) (end 172.76 101.75) (width 0.15) (layer "F.Cu") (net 6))
 (segment (start 172.525 105.635) (end 172.759651 105.635) (width 0.15) (layer "F.Cu") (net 6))
 (segment (start 171.93 102.5) (end 170.76 102.5) (width 0.15) (layer "F.Cu") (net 7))
 (segment (start 170.99 102.5) (end 171.74 101.75) (width 0.15) (layer "F.Cu") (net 7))
 (segment (start 172.525 103.095) (end 171.93 102.5) (width 0.15) (layer "F.Cu") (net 7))
 (segment (start 170.76 102.5) (end 170.99 102.5) (width 0.15) (layer "F.Cu") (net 7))
 (segment (start 170.76 107.5) (end 170.76 106.5) (width 0.15) (layer "F.Cu") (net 3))
 (segment (start 179.71548 108.04452) (end 171.30452 108.04452) (width 0.15) (layer "F.Cu") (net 3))
 (segment (start 171.30452 108.04452) (end 170.76 107.5) (width 0.15) (layer "F.Cu") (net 3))
 (segment (start 180.26 107.5) (end 179.71548 108.04452) (width 0.15) (layer "F.Cu") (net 3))
 (segment (start 177.475 106.905) (end 178.835 106.905) (width 0.15) (layer "F.Cu") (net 4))
 (segment (start 178.835 106.905) (end 179.24 106.5) (width 0.15) (layer "F.Cu") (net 4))
 (segment (start 179.24 107.5) (end 179.24 106.5) (width 0.15) (layer "F.Cu") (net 4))
 (segment (start 178.855 105.635) (end 179.24 105.25) (width 0.15) (layer "F.Cu") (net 11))
 (segment (start 179.26 105.25) (end 180.26 104.25) (width 0.15) (layer "F.Cu") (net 11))
 (segment (start 179.24 105.25) (end 179.26 105.25) (width 0.15) (layer "F.Cu") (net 11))
 (segment (start 177.475 105.635) (end 178.855 105.635) (width 0.15) (layer "F.Cu") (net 11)))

